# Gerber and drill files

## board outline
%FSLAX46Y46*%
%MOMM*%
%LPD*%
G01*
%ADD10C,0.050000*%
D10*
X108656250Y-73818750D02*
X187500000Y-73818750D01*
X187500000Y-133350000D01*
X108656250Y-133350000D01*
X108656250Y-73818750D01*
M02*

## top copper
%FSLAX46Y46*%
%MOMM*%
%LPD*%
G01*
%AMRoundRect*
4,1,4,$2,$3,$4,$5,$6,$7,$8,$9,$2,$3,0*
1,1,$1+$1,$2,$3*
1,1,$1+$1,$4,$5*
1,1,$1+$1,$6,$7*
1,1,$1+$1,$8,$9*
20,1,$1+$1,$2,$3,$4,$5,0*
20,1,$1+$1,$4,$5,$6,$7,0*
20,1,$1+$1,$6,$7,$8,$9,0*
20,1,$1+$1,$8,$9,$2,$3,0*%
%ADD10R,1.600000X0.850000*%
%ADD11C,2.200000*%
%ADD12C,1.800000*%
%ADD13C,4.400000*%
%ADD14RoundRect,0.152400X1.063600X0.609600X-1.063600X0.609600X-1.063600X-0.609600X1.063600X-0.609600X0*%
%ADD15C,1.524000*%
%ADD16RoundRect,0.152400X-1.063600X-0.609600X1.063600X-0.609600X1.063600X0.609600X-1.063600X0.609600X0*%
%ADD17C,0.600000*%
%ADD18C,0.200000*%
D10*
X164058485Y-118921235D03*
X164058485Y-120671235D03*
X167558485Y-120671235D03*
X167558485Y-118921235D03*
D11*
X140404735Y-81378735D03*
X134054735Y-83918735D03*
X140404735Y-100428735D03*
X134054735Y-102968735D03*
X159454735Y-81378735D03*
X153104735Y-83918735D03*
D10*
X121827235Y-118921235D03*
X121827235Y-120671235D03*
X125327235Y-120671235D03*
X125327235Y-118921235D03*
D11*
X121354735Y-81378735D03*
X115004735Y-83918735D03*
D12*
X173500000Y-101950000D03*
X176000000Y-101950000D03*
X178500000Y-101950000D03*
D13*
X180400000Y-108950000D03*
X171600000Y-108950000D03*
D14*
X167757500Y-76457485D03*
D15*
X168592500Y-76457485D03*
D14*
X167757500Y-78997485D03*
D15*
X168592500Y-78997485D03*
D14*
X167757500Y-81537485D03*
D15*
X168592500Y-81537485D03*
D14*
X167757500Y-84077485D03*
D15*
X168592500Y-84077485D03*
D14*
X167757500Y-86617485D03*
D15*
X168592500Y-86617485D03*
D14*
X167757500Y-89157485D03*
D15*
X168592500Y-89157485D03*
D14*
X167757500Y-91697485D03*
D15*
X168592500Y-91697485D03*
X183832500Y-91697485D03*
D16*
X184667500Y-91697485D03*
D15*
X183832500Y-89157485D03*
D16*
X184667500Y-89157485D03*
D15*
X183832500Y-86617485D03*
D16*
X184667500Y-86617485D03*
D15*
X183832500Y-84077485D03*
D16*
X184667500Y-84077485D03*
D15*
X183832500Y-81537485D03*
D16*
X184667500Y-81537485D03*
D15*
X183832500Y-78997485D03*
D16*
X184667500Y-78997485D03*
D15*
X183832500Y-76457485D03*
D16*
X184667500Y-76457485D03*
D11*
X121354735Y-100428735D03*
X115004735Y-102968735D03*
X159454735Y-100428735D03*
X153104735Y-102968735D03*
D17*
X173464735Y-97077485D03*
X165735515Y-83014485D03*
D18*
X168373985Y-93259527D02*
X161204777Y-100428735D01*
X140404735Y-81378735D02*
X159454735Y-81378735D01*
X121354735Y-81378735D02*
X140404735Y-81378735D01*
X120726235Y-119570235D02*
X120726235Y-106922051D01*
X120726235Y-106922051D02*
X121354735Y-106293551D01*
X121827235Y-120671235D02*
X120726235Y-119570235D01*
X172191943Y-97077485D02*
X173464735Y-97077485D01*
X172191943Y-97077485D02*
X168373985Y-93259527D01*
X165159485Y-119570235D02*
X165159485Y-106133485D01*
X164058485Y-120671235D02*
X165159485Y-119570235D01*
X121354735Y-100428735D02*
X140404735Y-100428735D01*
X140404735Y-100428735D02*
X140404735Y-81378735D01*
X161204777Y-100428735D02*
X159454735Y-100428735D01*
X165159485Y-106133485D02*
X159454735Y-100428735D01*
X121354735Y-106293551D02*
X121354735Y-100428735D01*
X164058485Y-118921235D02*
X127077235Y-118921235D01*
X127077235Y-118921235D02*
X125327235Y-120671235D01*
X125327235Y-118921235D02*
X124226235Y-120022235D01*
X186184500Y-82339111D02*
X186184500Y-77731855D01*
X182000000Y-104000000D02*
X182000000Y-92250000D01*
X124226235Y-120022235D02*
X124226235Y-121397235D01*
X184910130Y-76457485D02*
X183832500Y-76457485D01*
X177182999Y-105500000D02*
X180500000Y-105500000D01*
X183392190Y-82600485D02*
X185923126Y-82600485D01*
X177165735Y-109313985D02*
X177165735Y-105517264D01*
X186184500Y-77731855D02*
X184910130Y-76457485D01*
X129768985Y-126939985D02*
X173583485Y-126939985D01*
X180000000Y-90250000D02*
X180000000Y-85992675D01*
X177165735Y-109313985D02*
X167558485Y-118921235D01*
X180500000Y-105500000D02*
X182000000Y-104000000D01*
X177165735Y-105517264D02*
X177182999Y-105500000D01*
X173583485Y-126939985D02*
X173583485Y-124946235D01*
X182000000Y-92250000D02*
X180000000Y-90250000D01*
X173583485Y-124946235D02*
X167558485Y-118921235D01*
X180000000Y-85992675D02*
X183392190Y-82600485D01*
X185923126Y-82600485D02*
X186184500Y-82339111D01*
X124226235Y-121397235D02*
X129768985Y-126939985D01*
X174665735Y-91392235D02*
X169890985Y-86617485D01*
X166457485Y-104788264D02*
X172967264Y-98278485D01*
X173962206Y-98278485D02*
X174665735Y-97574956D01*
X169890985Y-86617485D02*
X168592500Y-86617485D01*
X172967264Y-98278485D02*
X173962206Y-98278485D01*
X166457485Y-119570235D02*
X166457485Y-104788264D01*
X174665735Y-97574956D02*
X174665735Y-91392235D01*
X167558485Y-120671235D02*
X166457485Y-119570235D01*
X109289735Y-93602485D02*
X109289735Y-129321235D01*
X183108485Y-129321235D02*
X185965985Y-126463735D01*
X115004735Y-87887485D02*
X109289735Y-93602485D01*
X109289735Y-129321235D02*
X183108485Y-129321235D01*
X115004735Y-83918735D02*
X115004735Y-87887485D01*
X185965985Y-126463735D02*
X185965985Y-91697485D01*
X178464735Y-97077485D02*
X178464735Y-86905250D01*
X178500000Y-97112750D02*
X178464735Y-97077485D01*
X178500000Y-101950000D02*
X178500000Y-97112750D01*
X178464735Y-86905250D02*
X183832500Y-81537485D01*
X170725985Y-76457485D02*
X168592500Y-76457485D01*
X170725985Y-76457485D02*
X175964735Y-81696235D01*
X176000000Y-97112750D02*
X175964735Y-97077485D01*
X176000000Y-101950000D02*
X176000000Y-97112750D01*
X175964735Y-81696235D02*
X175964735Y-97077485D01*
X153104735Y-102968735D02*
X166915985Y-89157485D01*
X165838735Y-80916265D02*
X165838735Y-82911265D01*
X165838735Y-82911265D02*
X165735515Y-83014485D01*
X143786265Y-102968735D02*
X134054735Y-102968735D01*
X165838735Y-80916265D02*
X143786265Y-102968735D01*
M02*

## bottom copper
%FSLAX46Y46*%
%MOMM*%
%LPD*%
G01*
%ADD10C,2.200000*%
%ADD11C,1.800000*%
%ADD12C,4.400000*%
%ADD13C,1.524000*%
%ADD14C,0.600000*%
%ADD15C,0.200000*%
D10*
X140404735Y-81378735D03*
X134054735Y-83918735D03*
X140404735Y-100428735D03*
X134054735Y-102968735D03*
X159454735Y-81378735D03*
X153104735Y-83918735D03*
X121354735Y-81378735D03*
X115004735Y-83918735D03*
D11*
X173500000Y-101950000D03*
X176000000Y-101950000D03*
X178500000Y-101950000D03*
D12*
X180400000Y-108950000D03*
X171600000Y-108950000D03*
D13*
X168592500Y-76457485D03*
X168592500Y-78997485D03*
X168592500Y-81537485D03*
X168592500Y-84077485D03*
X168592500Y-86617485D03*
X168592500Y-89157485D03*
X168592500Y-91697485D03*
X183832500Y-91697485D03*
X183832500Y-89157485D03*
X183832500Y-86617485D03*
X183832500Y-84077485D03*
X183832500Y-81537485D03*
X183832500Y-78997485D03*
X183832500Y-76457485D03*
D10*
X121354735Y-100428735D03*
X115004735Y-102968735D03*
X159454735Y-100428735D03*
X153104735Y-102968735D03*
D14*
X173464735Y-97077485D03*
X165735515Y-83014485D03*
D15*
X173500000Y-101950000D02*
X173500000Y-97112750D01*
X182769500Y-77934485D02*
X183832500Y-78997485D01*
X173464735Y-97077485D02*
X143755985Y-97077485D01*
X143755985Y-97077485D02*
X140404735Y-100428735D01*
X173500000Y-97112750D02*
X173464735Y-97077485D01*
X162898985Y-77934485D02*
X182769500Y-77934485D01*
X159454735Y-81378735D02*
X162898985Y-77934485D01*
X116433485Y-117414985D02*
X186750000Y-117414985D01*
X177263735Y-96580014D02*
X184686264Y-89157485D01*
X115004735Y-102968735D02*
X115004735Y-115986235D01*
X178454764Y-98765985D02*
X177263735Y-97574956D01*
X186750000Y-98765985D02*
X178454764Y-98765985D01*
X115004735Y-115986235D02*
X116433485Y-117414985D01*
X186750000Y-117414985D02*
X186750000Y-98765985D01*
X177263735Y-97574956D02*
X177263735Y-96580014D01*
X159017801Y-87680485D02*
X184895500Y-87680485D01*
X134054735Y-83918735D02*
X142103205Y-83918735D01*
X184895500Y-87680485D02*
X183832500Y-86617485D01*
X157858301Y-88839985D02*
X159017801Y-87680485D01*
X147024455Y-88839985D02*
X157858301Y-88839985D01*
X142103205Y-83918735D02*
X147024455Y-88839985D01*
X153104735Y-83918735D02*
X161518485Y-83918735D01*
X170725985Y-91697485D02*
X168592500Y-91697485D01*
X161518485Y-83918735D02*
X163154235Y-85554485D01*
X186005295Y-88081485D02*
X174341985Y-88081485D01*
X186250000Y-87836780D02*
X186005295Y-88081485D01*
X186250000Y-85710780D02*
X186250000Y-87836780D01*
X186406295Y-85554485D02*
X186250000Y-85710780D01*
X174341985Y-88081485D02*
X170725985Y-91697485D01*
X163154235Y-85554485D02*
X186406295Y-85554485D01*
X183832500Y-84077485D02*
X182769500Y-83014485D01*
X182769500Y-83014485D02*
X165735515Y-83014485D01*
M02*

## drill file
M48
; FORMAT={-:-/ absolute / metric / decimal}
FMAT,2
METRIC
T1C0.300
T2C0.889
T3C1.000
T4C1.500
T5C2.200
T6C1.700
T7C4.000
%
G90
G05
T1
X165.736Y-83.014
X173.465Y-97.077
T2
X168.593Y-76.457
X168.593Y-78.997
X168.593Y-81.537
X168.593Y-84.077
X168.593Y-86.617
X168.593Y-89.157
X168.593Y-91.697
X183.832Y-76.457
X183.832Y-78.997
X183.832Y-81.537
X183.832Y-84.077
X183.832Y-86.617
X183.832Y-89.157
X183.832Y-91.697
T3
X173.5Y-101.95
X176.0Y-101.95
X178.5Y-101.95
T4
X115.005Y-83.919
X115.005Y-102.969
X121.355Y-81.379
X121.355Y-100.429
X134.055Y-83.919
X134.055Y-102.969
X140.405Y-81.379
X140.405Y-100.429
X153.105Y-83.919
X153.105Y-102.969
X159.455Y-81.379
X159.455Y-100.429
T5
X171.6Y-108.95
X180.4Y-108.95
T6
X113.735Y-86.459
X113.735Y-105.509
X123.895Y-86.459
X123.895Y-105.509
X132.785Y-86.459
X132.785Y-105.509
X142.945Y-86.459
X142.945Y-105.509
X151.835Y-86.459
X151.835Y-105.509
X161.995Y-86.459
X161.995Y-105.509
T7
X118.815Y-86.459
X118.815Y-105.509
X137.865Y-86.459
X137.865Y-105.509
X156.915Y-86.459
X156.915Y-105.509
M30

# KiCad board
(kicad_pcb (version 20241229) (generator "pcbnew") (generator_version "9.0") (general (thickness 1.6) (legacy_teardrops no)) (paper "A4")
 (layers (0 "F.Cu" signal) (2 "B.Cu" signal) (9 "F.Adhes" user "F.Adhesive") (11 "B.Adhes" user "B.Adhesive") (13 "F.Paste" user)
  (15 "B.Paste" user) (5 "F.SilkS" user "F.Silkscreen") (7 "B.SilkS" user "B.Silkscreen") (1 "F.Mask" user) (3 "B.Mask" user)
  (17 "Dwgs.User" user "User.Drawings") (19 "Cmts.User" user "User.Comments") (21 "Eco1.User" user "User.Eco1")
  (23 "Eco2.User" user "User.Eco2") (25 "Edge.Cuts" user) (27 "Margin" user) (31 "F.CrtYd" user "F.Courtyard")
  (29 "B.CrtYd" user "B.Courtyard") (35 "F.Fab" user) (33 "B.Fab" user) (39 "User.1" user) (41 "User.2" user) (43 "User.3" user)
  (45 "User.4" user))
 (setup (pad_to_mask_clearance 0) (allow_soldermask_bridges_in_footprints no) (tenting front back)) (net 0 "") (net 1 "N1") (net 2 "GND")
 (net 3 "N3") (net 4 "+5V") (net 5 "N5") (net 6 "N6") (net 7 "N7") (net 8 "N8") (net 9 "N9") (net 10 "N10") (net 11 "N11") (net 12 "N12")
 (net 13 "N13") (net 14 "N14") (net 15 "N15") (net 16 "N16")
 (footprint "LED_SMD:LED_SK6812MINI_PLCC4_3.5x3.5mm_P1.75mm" (layer "F.Cu") (at 165.808485 119.796235)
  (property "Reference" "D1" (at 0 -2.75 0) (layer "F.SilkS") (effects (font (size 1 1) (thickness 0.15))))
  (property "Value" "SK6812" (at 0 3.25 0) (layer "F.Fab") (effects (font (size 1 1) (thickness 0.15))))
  (pad "1" smd rect (at -1.75 -0.875) (size 1.6 0.85) (layers "F.Cu" "F.Mask" "F.Paste") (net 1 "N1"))
  (pad "2" smd rect (at -1.75 0.875) (size 1.6 0.85) (layers "F.Cu" "F.Mask" "F.Paste") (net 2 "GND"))
  (pad "3" smd rect (at 1.75 0.875) (size 1.6 0.85) (layers "F.Cu" "F.Mask" "F.Paste") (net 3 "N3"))
  (pad "4" smd rect (at 1.75 -0.875) (size 1.6 0.85) (layers "F.Cu" "F.Mask" "F.Paste") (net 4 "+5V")))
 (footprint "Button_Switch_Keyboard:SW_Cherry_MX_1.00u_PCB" (layer "F.Cu") (at 140.404735 81.378735)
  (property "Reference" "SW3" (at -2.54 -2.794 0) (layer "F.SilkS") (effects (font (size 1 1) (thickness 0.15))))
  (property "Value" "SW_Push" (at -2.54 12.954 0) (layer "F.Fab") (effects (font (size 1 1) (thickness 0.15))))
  (pad "" np_thru_hole circle (at -7.62 5.08) (size 1.7 1.7) (drill 1.7) (layers "*.Cu" "*.Mask"))
  (pad "" np_thru_hole circle (at -2.54 5.08) (size 4 4) (drill 4) (layers "*.Cu" "*.Mask"))
  (pad "" np_thru_hole circle (at 2.54 5.08) (size 1.7 1.7) (drill 1.7) (layers "*.Cu" "*.Mask"))
  (pad "1" thru_hole circle (at 0 0) (size 2.2 2.2) (drill 1.5) (layers "*.Cu" "*.Mask") (remove_unused_layers no) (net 2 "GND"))
  (pad "2" thru_hole circle (at -6.35 2.54) (size 2.2 2.2) (drill 1.5) (layers "*.Cu" "*.Mask") (remove_unused_layers no) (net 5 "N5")))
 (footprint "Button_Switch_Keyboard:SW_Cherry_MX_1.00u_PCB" (layer "F.Cu") (at 140.404735 100.428735)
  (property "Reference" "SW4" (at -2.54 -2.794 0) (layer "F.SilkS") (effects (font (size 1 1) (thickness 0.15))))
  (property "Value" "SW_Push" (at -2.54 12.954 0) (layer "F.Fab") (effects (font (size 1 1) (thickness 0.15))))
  (pad "" np_thru_hole circle (at -7.62 5.08) (size 1.7 1.7) (drill 1.7) (layers "*.Cu" "*.Mask"))
  (pad "" np_thru_hole circle (at -2.54 5.08) (size 4 4) (drill 4) (layers "*.Cu" "*.Mask"))
  (pad "" np_thru_hole circle (at 2.54 5.08) (size 1.7 1.7) (drill 1.7) (layers "*.Cu" "*.Mask"))
  (pad "1" thru_hole circle (at 0 0) (size 2.2 2.2) (drill 1.5) (layers "*.Cu" "*.Mask") (remove_unused_layers no) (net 2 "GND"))
  (pad "2" thru_hole circle (at -6.35 2.54) (size 2.2 2.2) (drill 1.5) (layers "*.Cu" "*.Mask") (remove_unused_layers no) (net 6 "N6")))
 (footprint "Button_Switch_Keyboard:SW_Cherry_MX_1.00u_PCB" (layer "F.Cu") (at 159.454735 81.378735)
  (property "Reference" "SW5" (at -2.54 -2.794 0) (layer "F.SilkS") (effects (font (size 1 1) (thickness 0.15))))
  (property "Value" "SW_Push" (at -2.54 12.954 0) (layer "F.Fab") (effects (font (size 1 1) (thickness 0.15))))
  (pad "" np_thru_hole circle (at -7.62 5.08) (size 1.7 1.7) (drill 1.7) (layers "*.Cu" "*.Mask"))
  (pad "" np_thru_hole circle (at -2.54 5.08) (size 4 4) (drill 4) (layers "*.Cu" "*.Mask"))
  (pad "" np_thru_hole circle (at 2.54 5.08) (size 1.7 1.7) (drill 1.7) (layers "*.Cu" "*.Mask"))
  (pad "1" thru_hole circle (at 0 0) (size 2.2 2.2) (drill 1.5) (layers "*.Cu" "*.Mask") (remove_unused_layers no) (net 2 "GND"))
  (pad "2" thru_hole circle (at -6.35 2.54) (size 2.2 2.2) (drill 1.5) (layers "*.Cu" "*.Mask") (remove_unused_layers no) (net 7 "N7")))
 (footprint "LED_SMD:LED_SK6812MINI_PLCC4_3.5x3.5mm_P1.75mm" (layer "F.Cu") (at 123.577235 119.796235)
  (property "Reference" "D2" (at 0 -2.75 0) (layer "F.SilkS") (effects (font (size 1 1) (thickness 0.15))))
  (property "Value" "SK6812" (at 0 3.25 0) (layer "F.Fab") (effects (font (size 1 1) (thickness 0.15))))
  (pad "1" smd rect (at -1.75 -0.875) (size 1.6 0.85) (layers "F.Cu" "F.Mask" "F.Paste") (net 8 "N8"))
  (pad "2" smd rect (at -1.75 0.875) (size 1.6 0.85) (layers "F.Cu" "F.Mask" "F.Paste") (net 2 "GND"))
  (pad "3" smd rect (at 1.75 0.875) (size 1.6 0.85) (layers "F.Cu" "F.Mask" "F.Paste") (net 1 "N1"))
  (pad "4" smd rect (at 1.75 -0.875) (size 1.6 0.85) (layers "F.Cu" "F.Mask" "F.Paste") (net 4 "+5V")))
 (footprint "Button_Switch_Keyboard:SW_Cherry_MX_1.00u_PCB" (layer "F.Cu") (at 121.354735 81.378735)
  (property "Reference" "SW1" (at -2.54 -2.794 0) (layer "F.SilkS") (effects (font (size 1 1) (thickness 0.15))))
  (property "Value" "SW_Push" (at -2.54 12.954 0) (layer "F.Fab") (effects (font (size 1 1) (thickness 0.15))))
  (pad "" np_thru_hole circle (at -7.62 5.08) (size 1.7 1.7) (drill 1.7) (layers "*.Cu" "*.Mask"))
  (pad "" np_thru_hole circle (at -2.54 5.08) (size 4 4) (drill 4) (layers "*.Cu" "*.Mask"))
  (pad "" np_thru_hole circle (at 2.54 5.08) (size 1.7 1.7) (drill 1.7) (layers "*.Cu" "*.Mask"))
  (pad "1" thru_hole circle (at 0 0) (size 2.2 2.2) (drill 1.5) (layers "*.Cu" "*.Mask") (remove_unused_layers no) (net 2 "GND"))
  (pad "2" thru_hole circle (at -6.35 2.54) (size 2.2 2.2) (drill 1.5) (layers "*.Cu" "*.Mask") (remove_unused_layers no) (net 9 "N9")))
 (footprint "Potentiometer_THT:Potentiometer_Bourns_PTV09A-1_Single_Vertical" (layer "F.Cu") (at 173.5 101.95 -90)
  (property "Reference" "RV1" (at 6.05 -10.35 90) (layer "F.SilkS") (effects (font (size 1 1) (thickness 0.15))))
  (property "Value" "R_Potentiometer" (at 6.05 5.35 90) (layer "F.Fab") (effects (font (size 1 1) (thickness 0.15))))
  (pad "1" thru_hole circle (at 0 0 270) (size 1.8 1.8) (drill 1) (layers "*.Cu" "*.Mask") (remove_unused_layers no) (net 2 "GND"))
  (pad "2" thru_hole circle (at 0 -2.5 270) (size 1.8 1.8) (drill 1) (layers "*.Cu" "*.Mask") (remove_unused_layers no) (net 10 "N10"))
  (pad "3" thru_hole circle (at 0 -5 270) (size 1.8 1.8) (drill 1) (layers "*.Cu" "*.Mask") (remove_unused_layers no) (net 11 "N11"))
  (pad "MP" thru_hole circle (at 7 -6.9 270) (size 4.4 4.4) (drill 2.2) (layers "*.Cu" "*.Mask") (remove_unused_layers no))
  (pad "MP" thru_hole circle (at 7 1.9 270) (size 4.4 4.4) (drill 2.2) (layers "*.Cu" "*.Mask") (remove_unused_layers no)))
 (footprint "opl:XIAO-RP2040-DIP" (layer "F.Cu") (at 176.2125 84.077485)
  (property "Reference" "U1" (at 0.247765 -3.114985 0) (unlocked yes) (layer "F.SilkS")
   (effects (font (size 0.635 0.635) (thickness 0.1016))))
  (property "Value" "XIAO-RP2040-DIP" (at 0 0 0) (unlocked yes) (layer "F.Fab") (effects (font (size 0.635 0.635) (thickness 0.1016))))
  (pad "1" smd roundrect (at -8.455 -7.62 180) (size 2.432 1.524) (layers "F.Cu" "F.Mask") (roundrect_rratio 0.1) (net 10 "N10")
   (thermal_bridge_angle 45))
  (pad "1" thru_hole circle (at -7.62 -7.62 180) (size 1.524 1.524) (drill 0.889) (layers "*.Cu" "*.Mask") (remove_unused_layers no)
   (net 10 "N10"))
  (pad "2" smd roundrect (at -8.455 -5.08 180) (size 2.432 1.524) (layers "F.Cu" "F.Mask") (roundrect_rratio 0.1) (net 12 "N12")
   (thermal_bridge_angle 45))
  (pad "2" thru_hole circle (at -7.62 -5.08 180) (size 1.524 1.524) (drill 0.889) (layers "*.Cu" "*.Mask") (remove_unused_layers no)
   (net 12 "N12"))
  (pad "3" smd roundrect (at -8.455 -2.54 180) (size 2.432 1.524) (layers "F.Cu" "F.Mask") (roundrect_rratio 0.1) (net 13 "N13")
   (thermal_bridge_angle 45))
  (pad "3" thru_hole circle (at -7.62 -2.54 180) (size 1.524 1.524) (drill 0.889) (layers "*.Cu" "*.Mask") (remove_unused_layers no)
   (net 13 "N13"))
  (pad "4" smd roundrect (at -8.455 0 180) (size 2.432 1.524) (layers "F.Cu" "F.Mask") (roundrect_rratio 0.1) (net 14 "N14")
   (thermal_bridge_angle 45))
  (pad "4" thru_hole circle (at -7.62 0 180) (size 1.524 1.524) (drill 0.889) (layers "*.Cu" "*.Mask") (remove_unused_layers no)
   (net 14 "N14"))
  (pad "5" smd roundrect (at -8.455 2.54 180) (size 2.432 1.524) (layers "F.Cu" "F.Mask") (roundrect_rratio 0.1) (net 3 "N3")
   (thermal_bridge_angle 45))
  (pad "5" thru_hole circle (at -7.62 2.54 180) (size 1.524 1.524) (drill 0.889) (layers "*.Cu" "*.Mask") (remove_unused_layers no)
   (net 3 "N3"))
  (pad "6" smd roundrect (at -8.455 5.08 180) (size 2.432 1.524) (layers "F.Cu" "F.Mask") (roundrect_rratio 0.1) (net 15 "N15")
   (thermal_bridge_angle 45))
  (pad "6" thru_hole circle (at -7.62 5.08 180) (size 1.524 1.524) (drill 0.889) (layers "*.Cu" "*.Mask") (remove_unused_layers no)
   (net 15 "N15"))
  (pad "7" smd roundrect (at -8.455 7.62 180) (size 2.432 1.524) (layers "F.Cu" "F.Mask") (roundrect_rratio 0.1) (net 7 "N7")
   (thermal_bridge_angle 45))
  (pad "7" thru_hole circle (at -7.62 7.62 180) (size 1.524 1.524) (drill 0.889) (layers "*.Cu" "*.Mask") (remove_unused_layers no)
   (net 7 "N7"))
  (pad "8" thru_hole circle (at 7.62 7.62) (size 1.524 1.524) (drill 0.889) (layers "*.Cu" "*.Mask") (remove_unused_layers no) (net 9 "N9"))
  (pad "8" smd roundrect (at 8.455 7.62) (size 2.432 1.524) (layers "F.Cu" "F.Mask") (roundrect_rratio 0.1) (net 9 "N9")
   (thermal_bridge_angle 45))
  (pad "9" thru_hole circle (at 7.62 5.08) (size 1.524 1.524) (drill 0.889) (layers "*.Cu" "*.Mask") (remove_unused_layers no)
   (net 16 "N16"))
  (pad "9" smd roundrect (at 8.455 5.08) (size 2.432 1.524) (layers "F.Cu" "F.Mask") (roundrect_rratio 0.1) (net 16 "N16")
   (thermal_bridge_angle 45))
  (pad "10" thru_hole circle (at 7.62 2.54) (size 1.524 1.524) (drill 0.889) (layers "*.Cu" "*.Mask") (remove_unused_layers no) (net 5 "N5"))
  (pad "10" smd roundrect (at 8.455 2.54) (size 2.432 1.524) (layers "F.Cu" "F.Mask") (roundrect_rratio 0.1) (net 5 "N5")
   (thermal_bridge_angle 45))
  (pad "11" thru_hole circle (at 7.62 0) (size 1.524 1.524) (drill 0.889) (layers "*.Cu" "*.Mask") (remove_unused_layers no) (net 6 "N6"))
  (pad "11" smd roundrect (at 8.455 0) (size 2.432 1.524) (layers "F.Cu" "F.Mask") (roundrect_rratio 0.1) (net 6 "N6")
   (thermal_bridge_angle 45))
  (pad "12" thru_hole circle (at 7.62 -2.54) (size 1.524 1.524) (drill 0.889) (layers "*.Cu" "*.Mask") (remove_unused_layers no)
   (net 11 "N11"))
  (pad "12" smd roundrect (at 8.455 -2.54) (size 2.432 1.524) (layers "F.Cu" "F.Mask") (roundrect_rratio 0.1) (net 11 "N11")
   (thermal_bridge_angle 45))
  (pad "13" thru_hole circle (at 7.62 -5.08) (size 1.524 1.524) (drill 0.889) (layers "*.Cu" "*.Mask") (remove_unused_layers no)
   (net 2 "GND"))
  (pad "13" smd roundrect (at 8.455 -5.08) (size 2.432 1.524) (layers "F.Cu" "F.Mask") (roundrect_rratio 0.1) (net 2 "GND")
   (thermal_bridge_angle 45))
  (pad "14" thru_hole circle (at 7.62 -7.62) (size 1.524 1.524) (drill 0.889) (layers "*.Cu" "*.Mask") (remove_unused_layers no)
   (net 4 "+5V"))
  (pad "14" smd roundrect (at 8.455 -7.62) (size 2.432 1.524) (layers "F.Cu" "F.Mask") (roundrect_rratio 0.1) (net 4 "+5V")
   (thermal_bridge_angle 45)))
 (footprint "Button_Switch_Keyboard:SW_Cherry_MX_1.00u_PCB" (layer "F.Cu") (at 121.354735 100.428735)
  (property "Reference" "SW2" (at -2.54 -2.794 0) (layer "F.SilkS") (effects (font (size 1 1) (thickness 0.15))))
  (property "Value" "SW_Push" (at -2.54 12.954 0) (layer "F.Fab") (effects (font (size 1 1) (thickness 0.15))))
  (pad "" np_thru_hole circle (at -7.62 5.08) (size 1.7 1.7) (drill 1.7) (layers "*.Cu" "*.Mask"))
  (pad "" np_thru_hole circle (at -2.54 5.08) (size 4 4) (drill 4) (layers "*.Cu" "*.Mask"))
  (pad "" np_thru_hole circle (at 2.54 5.08) (size 1.7 1.7) (drill 1.7) (layers "*.Cu" "*.Mask"))
  (pad "1" thru_hole circle (at 0 0) (size 2.2 2.2) (drill 1.5) (layers "*.Cu" "*.Mask") (remove_unused_layers no) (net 2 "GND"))
  (pad "2" thru_hole circle (at -6.35 2.54) (size 2.2 2.2) (drill 1.5) (layers "*.Cu" "*.Mask") (remove_unused_layers no) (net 16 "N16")))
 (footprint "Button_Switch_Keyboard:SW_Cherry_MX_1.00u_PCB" (layer "F.Cu") (at 159.454735 100.428735)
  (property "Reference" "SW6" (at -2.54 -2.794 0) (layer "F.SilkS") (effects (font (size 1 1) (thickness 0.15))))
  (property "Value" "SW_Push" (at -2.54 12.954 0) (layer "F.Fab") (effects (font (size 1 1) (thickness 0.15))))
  (pad "" np_thru_hole circle (at -7.62 5.08) (size 1.7 1.7) (drill 1.7) (layers "*.Cu" "*.Mask"))
  (pad "" np_thru_hole circle (at -2.54 5.08) (size 4 4) (drill 4) (layers "*.Cu" "*.Mask"))
  (pad "" np_thru_hole circle (at 2.54 5.08) (size 1.7 1.7) (drill 1.7) (layers "*.Cu" "*.Mask"))
  (pad "1" thru_hole circle (at 0 0) (size 2.2 2.2) (drill 1.5) (layers "*.Cu" "*.Mask") (remove_unused_layers no) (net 2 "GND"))
  (pad "2" thru_hole circle (at -6.35 2.54) (size 2.2 2.2) (drill 1.5) (layers "*.Cu" "*.Mask") (remove_unused_layers no) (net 15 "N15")))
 (gr_rect (start 108.65625 73.81875) (end 187.5 133.35) (stroke (width 0.05) (type default)) (fill no) (layer "Edge.Cuts"))
 (segment (start 168.373985 93.259527) (end 161.204777 100.428735) (width 0.2) (layer "F.Cu") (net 2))
 (segment (start 140.404735 81.378735) (end 159.454735 81.378735) (width 0.2) (layer "F.Cu") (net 2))
 (segment (start 121.354735 81.378735) (end 140.404735 81.378735) (width 0.2) (layer "F.Cu") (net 2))
 (segment (start 120.726235 119.570235) (end 120.726235 106.922051) (width 0.2) (layer "F.Cu") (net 2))
 (segment (start 120.726235 106.922051) (end 121.354735 106.293551) (width 0.2) (layer "F.Cu") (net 2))
 (segment (start 121.827235 120.671235) (end 120.726235 119.570235) (width 0.2) (layer "F.Cu") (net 2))
 (segment (start 172.191943 97.077485) (end 173.464735 97.077485) (width 0.2) (layer "F.Cu") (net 2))
 (segment (start 172.191943 97.077485) (end 168.373985 93.259527) (width 0.2) (layer "F.Cu") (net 2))
 (segment (start 165.159485 119.570235) (end 165.159485 106.133485) (width 0.2) (layer "F.Cu") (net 2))
 (segment (start 164.058485 120.671235) (end 165.159485 119.570235) (width 0.2) (layer "F.Cu") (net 2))
 (segment (start 121.354735 100.428735) (end 140.404735 100.428735) (width 0.2) (layer "F.Cu") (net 2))
 (segment (start 140.404735 100.428735) (end 140.404735 81.378735) (width 0.2) (layer "F.Cu") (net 2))
 (segment (start 161.204777 100.428735) (end 159.454735 100.428735) (width 0.2) (layer "F.Cu") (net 2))
 (segment (start 165.159485 106.133485) (end 159.454735 100.428735) (width 0.2) (layer "F.Cu") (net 2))
 (segment (start 121.354735 106.293551) (end 121.354735 100.428735) (width 0.2) (layer "F.Cu") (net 2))
 (via (at 173.464735 97.077485) (size 0.6) (drill 0.3) (layers "F.Cu" "B.Cu") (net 2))
 (segment (start 173.5 101.95) (end 173.5 97.11275) (width 0.2) (layer "B.Cu") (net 2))
 (segment (start 182.7695 77.934485) (end 183.8325 78.997485) (width 0.2) (layer "B.Cu") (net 2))
 (segment (start 173.464735 97.077485) (end 143.755985 97.077485) (width 0.2) (layer "B.Cu") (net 2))
 (segment (start 143.755985 97.077485) (end 140.404735 100.428735) (width 0.2) (layer "B.Cu") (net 2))
 (segment (start 173.5 97.11275) (end 173.464735 97.077485) (width 0.2) (layer "B.Cu") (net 2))
 (segment (start 162.898985 77.934485) (end 182.7695 77.934485) (width 0.2) (layer "B.Cu") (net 2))
 (segment (start 159.454735 81.378735) (end 162.898985 77.934485) (width 0.2) (layer "B.Cu") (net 2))
 (segment (start 164.058485 118.921235) (end 127.077235 118.921235) (width 0.2) (layer "F.Cu") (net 1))
 (segment (start 127.077235 118.921235) (end 125.327235 120.671235) (width 0.2) (layer "F.Cu") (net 1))
 (segment (start 125.327235 118.921235) (end 124.226235 120.022235) (width 0.2) (layer "F.Cu") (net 4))
 (segment (start 186.1845 82.339111) (end 186.1845 77.731855) (width 0.2) (layer "F.Cu") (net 4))
 (segment (start 182 104) (end 182 92.25) (width 0.2) (layer "F.Cu") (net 4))
 (segment (start 124.226235 120.022235) (end 124.226235 121.397235) (width 0.2) (layer "F.Cu") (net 4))
 (segment (start 184.91013 76.457485) (end 183.8325 76.457485) (width 0.2) (layer "F.Cu") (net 4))
 (segment (start 177.182999 105.5) (end 180.5 105.5) (width 0.2) (layer "F.Cu") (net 4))
 (segment (start 183.39219 82.600485) (end 185.923126 82.600485) (width 0.2) (layer "F.Cu") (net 4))
 (segment (start 177.165735 109.313985) (end 177.165735 105.517264) (width 0.2) (layer "F.Cu") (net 4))
 (segment (start 186.1845 77.731855) (end 184.91013 76.457485) (width 0.2) (layer "F.Cu") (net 4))
 (segment (start 129.768985 126.939985) (end 173.583485 126.939985) (width 0.2) (layer "F.Cu") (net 4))
 (segment (start 180 90.25) (end 180 85.992675) (width 0.2) (layer "F.Cu") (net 4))
 (segment (start 177.165735 109.313985) (end 167.558485 118.921235) (width 0.2) (layer "F.Cu") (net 4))
 (segment (start 180.5 105.5) (end 182 104) (width 0.2) (layer "F.Cu") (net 4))
 (segment (start 177.165735 105.517264) (end 177.182999 105.5) (width 0.2) (layer "F.Cu") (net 4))
 (segment (start 173.583485 126.939985) (end 173.583485 124.946235) (width 0.2) (layer "F.Cu") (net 4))
 (segment (start 182 92.25) (end 180 90.25) (width 0.2) (layer "F.Cu") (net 4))
 (segment (start 173.583485 124.946235) (end 167.558485 118.921235) (width 0.2) (layer "F.Cu") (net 4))
 (segment (start 180 85.992675) (end 183.39219 82.600485) (width 0.2) (layer "F.Cu") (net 4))
 (segment (start 185.923126 82.600485) (end 186.1845 82.339111) (width 0.2) (layer "F.Cu") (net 4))
 (segment (start 124.226235 121.397235) (end 129.768985 126.939985) (width 0.2) (layer "F.Cu") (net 4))
 (segment (start 174.665735 91.392235) (end 169.890985 86.617485) (width 0.2) (layer "F.Cu") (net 3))
 (segment (start 166.457485 104.788264) (end 172.967264 98.278485) (width 0.2) (layer "F.Cu") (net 3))
 (segment (start 173.962206 98.278485) (end 174.665735 97.574956) (width 0.2) (layer "F.Cu") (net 3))
 (segment (start 169.890985 86.617485) (end 168.5925 86.617485) (width 0.2) (layer "F.Cu") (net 3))
 (segment (start 172.967264 98.278485) (end 173.962206 98.278485) (width 0.2) (layer "F.Cu") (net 3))
 (segment (start 166.457485 119.570235) (end 166.457485 104.788264) (width 0.2) (layer "F.Cu") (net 3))
 (segment (start 174.665735 97.574956) (end 174.665735 91.392235) (width 0.2) (layer "F.Cu") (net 3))
 (segment (start 167.558485 120.671235) (end 166.457485 119.570235) (width 0.2) (layer "F.Cu") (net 3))
 (segment (start 109.289735 93.602485) (end 109.289735 129.321235) (width 0.2) (layer "F.Cu") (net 9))
 (segment (start 183.108485 129.321235) (end 185.965985 126.463735) (width 0.2) (layer "F.Cu") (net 9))
 (segment (start 115.004735 87.887485) (end 109.289735 93.602485) (width 0.2) (layer "F.Cu") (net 9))
 (segment (start 109.289735 129.321235) (end 183.108485 129.321235) (width 0.2) (layer "F.Cu") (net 9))
 (segment (start 115.004735 83.918735) (end 115.004735 87.887485) (width 0.2) (layer "F.Cu") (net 9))
 (segment (start 185.965985 126.463735) (end 185.965985 91.697485) (width 0.2) (layer "F.Cu") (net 9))
 (segment (start 116.433485 117.414985) (end 186.75 117.414985) (width 0.2) (layer "B.Cu") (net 16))
 (segment (start 177.263735 96.580014) (end 184.686264 89.157485) (width 0.2) (layer "B.Cu") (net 16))
 (segment (start 115.004735 102.968735) (end 115.004735 115.986235) (width 0.2) (layer "B.Cu") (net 16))
 (segment (start 178.454764 98.765985) (end 177.263735 97.574956) (width 0.2) (layer "B.Cu") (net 16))
 (segment (start 186.75 98.765985) (end 178.454764 98.765985) (width 0.2) (layer "B.Cu") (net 16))
 (segment (start 115.004735 115.986235) (end 116.433485 117.414985) (width 0.2) (layer "B.Cu") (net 16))
 (segment (start 186.75 117.414985) (end 186.75 98.765985) (width 0.2) (layer "B.Cu") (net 16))
 (segment (start 177.263735 97.574956) (end 177.263735 96.580014) (width 0.2) (layer "B.Cu") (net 16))
 (segment (start 159.017801 87.680485) (end 184.8955 87.680485) (width 0.2) (layer "B.Cu") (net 5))
 (segment (start 134.054735 83.918735) (end 142.103205 83.918735) (width 0.2) (layer "B.Cu") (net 5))
 (segment (start 184.8955 87.680485) (end 183.8325 86.617485) (width 0.2) (layer "B.Cu") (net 5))
 (segment (start 157.858301 88.839985) (end 159.017801 87.680485) (width 0.2) (layer "B.Cu") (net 5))
 (segment (start 147.024455 88.839985) (end 157.858301 88.839985) (width 0.2) (layer "B.Cu") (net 5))
 (segment (start 142.103205 83.918735) (end 147.024455 88.839985) (width 0.2) (layer "B.Cu") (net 5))
 (segment (start 178.464735 97.077485) (end 178.464735 86.90525) (width 0.2) (layer "F.Cu") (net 11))
 (segment (start 178.5 97.11275) (end 178.464735 97.077485) (width 0.2) (layer "F.Cu") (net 11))
 (segment (start 178.5 101.95) (end 178.5 97.11275) (width 0.2) (layer "F.Cu") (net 11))
 (segment (start 178.464735 86.90525) (end 183.8325 81.537485) (width 0.2) (layer "F.Cu") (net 11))
 (segment (start 170.725985 76.457485) (end 168.5925 76.457485) (width 0.2) (layer "F.Cu") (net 10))
 (segment (start 170.725985 76.457485) (end 175.964735 81.696235) (width 0.2) (layer "F.Cu") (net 10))
 (segment (start 176 97.11275) (end 175.964735 97.077485) (width 0.2) (layer "F.Cu") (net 10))
 (segment (start 176 101.95) (end 176 97.11275) (width 0.2) (layer "F.Cu") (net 10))
 (segment (start 175.964735 81.696235) (end 175.964735 97.077485) (width 0.2) (layer "F.Cu") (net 10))
 (segment (start 153.104735 83.918735) (end 161.518485 83.918735) (width 0.2) (layer "B.Cu") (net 7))
 (segment (start 170.725985 91.697485) (end 168.5925 91.697485) (width 0.2) (layer "B.Cu") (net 7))
 (segment (start 161.518485 83.918735) (end 163.154235 85.554485) (width 0.2) (layer "B.Cu") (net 7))
 (segment (start 186.005295 88.081485) (end 174.341985 88.081485) (width 0.2) (layer "B.Cu") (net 7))
 (segment (start 186.25 87.83678) (end 186.005295 88.081485) (width 0.2) (layer "B.Cu") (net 7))
 (segment (start 186.25 85.71078) (end 186.25 87.83678) (width 0.2) (layer "B.Cu") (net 7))
 (segment (start 186.406295 85.554485) (end 186.25 85.71078) (width 0.2) (layer "B.Cu") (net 7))
 (segment (start 174.341985 88.081485) (end 170.725985 91.697485) (width 0.2) (layer "B.Cu") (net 7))
 (segment (start 163.154235 85.554485) (end 186.406295 85.554485) (width 0.2) (layer "B.Cu") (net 7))
 (segment (start 153.104735 102.968735) (end 166.915985 89.157485) (width 0.2) (layer "F.Cu") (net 15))
 (segment (start 165.838735 80.916265) (end 165.838735 82.911265) (width 0.2) (layer "F.Cu") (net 6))
 (segment (start 165.838735 82.911265) (end 165.735515 83.014485) (width 0.2) (layer "F.Cu") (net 6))
 (segment (start 143.786265 102.968735) (end 134.054735 102.968735) (width 0.2) (layer "F.Cu") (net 6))
 (segment (start 165.838735 80.916265) (end 143.786265 102.968735) (width 0.2) (layer "F.Cu") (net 6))
 (via (at 165.735515 83.014485) (size 0.6) (drill 0.3) (layers "F.Cu" "B.Cu") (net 6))
 (segment (start 183.8325 84.077485) (end 182.7695 83.014485) (width 0.2) (layer "B.Cu") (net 6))
 (segment (start 182.7695 83.014485) (end 165.735515 83.014485) (width 0.2) (layer "B.Cu") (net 6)))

